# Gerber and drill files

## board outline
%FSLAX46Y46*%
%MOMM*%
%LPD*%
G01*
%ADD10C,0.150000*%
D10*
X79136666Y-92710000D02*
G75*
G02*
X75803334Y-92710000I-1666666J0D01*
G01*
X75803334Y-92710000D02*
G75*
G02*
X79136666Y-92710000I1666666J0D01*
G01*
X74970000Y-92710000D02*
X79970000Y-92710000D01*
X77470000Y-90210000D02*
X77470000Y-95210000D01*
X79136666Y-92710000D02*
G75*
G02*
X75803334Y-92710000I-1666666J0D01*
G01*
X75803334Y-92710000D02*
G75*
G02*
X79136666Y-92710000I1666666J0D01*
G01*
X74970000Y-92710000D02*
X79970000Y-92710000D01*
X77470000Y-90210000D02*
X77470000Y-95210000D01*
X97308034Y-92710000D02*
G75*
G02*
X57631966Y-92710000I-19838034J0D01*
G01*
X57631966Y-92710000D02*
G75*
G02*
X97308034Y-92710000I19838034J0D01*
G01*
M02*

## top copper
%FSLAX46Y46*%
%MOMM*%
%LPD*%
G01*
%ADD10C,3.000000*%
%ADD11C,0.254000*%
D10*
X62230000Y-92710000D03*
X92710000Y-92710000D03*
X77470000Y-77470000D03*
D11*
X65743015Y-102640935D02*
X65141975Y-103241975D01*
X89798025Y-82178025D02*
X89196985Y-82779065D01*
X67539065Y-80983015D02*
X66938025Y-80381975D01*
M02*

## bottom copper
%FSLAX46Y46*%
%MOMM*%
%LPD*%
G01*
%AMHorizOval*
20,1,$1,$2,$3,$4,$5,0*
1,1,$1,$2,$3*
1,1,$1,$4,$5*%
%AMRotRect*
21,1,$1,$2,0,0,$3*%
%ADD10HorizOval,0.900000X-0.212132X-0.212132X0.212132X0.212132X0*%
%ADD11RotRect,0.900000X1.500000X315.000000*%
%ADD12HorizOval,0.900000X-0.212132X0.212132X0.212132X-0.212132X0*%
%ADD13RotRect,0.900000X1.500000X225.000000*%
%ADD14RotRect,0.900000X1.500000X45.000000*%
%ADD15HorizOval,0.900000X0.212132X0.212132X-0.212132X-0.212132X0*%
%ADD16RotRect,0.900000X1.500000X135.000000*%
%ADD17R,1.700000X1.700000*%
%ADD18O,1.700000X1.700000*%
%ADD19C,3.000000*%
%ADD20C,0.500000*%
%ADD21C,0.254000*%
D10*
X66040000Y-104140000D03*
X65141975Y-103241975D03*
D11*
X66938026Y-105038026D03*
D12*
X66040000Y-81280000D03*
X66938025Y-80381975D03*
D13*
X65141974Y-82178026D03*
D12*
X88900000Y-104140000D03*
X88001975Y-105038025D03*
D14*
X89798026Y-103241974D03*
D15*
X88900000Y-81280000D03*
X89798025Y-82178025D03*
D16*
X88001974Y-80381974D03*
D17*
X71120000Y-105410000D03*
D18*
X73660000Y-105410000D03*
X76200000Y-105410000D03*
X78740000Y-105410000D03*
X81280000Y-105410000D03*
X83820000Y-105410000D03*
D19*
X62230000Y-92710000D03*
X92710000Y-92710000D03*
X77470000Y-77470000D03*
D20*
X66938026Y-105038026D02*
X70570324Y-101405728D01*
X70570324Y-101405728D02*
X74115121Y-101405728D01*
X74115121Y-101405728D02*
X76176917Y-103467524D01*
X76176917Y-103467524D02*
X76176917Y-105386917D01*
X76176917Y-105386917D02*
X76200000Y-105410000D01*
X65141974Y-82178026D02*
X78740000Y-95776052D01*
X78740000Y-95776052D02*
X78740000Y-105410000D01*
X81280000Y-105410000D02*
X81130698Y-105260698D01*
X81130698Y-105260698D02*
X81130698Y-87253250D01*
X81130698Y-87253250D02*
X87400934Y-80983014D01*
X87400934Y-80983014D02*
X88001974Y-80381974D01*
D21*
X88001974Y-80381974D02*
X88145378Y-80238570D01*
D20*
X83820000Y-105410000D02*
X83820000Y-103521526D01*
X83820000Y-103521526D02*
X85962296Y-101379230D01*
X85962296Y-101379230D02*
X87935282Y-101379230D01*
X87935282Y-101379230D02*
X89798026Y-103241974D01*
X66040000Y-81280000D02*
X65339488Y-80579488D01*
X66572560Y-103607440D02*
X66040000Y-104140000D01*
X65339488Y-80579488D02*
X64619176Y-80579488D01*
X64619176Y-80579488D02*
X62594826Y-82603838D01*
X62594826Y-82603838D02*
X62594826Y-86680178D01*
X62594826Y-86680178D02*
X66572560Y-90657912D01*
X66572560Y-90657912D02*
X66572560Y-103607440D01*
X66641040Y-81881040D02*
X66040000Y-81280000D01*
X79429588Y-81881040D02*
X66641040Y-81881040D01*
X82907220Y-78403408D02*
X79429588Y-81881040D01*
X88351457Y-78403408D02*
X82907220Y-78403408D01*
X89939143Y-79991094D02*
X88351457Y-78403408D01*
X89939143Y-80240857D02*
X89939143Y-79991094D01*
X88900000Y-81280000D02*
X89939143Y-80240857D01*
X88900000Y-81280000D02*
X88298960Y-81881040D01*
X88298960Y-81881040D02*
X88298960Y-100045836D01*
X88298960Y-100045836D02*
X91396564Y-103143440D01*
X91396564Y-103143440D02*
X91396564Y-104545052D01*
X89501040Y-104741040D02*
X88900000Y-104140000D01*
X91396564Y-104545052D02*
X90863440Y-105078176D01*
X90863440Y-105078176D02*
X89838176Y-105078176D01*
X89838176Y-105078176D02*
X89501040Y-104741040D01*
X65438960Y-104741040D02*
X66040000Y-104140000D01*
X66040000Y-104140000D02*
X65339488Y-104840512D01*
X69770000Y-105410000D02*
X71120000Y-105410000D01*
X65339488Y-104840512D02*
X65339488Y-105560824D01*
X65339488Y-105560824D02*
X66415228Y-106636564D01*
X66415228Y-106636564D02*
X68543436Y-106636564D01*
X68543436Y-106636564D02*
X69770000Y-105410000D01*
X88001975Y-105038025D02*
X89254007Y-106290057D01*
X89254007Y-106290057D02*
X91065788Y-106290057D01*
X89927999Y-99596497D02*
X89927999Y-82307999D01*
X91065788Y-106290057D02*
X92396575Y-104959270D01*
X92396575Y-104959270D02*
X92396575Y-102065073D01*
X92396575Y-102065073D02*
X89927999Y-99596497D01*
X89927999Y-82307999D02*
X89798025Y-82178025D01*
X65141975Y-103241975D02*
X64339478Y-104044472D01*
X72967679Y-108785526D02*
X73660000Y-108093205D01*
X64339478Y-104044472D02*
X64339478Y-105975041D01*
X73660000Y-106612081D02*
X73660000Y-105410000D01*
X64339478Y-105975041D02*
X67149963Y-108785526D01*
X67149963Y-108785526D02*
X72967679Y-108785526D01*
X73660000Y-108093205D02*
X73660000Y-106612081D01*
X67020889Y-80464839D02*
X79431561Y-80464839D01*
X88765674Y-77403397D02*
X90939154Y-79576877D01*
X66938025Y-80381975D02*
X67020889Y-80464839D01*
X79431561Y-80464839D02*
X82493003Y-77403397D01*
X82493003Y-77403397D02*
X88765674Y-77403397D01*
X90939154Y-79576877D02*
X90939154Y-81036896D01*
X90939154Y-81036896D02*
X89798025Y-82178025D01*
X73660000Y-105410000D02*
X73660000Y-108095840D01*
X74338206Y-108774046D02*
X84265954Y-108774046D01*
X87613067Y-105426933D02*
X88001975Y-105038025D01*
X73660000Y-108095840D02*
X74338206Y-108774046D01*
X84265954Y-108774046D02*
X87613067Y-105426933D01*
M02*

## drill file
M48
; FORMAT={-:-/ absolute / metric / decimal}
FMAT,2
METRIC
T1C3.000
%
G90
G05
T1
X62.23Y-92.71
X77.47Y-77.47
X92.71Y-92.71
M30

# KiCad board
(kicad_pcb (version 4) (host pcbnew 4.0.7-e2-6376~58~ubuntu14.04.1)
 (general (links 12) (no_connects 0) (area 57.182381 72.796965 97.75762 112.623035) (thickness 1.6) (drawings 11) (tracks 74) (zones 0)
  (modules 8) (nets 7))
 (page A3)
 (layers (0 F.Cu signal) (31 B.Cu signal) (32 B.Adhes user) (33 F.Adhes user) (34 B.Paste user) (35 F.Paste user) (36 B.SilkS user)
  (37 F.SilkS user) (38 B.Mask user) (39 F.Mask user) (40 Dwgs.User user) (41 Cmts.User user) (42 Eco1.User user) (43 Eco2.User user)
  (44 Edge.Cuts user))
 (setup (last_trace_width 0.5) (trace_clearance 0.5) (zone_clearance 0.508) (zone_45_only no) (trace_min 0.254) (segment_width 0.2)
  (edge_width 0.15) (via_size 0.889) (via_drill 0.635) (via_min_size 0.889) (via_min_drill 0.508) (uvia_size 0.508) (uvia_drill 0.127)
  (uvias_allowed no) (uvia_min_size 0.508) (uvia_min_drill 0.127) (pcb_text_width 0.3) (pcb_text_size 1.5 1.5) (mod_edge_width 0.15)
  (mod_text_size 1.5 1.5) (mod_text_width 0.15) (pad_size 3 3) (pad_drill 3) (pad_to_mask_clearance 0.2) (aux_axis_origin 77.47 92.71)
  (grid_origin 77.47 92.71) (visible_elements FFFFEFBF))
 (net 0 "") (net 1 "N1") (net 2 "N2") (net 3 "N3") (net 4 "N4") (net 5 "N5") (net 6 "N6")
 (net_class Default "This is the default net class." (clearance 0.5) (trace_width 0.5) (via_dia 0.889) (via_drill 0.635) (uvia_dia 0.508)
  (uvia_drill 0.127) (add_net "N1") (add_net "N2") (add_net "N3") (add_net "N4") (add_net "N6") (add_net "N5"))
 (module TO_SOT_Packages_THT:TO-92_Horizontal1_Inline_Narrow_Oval (layer F.Cu) (at 66.938026 105.038026 135)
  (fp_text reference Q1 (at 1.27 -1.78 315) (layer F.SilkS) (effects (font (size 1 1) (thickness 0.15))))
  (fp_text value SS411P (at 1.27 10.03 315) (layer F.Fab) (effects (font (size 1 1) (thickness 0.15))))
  (pad 2 smd oval (at 1.270001 0 315) (size 0.9 1.5) (layers B.Cu F.Paste F.Mask) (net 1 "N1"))
  (pad 3 smd oval (at 2.54 0 315) (size 0.9 1.5) (layers B.Cu F.Paste F.Mask) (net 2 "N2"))
  (pad 1 smd rect (at 0 0 315) (size 0.9 1.5) (layers B.Cu F.Paste F.Mask) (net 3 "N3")))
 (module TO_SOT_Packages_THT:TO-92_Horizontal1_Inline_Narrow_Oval (layer F.Cu) (at 65.141974 82.178026 45)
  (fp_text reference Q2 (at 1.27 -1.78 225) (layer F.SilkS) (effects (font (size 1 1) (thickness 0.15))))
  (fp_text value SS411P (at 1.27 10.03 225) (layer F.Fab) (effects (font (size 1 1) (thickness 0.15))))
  (pad 2 smd oval (at 1.270001 0 225) (size 0.9 1.5) (layers B.Cu F.Paste F.Mask) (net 1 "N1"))
  (pad 3 smd oval (at 2.54 0 225) (size 0.9 1.5) (layers B.Cu F.Paste F.Mask) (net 2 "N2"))
  (pad 1 smd rect (at 0 0 225) (size 0.9 1.5) (layers B.Cu F.Paste F.Mask) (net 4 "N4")))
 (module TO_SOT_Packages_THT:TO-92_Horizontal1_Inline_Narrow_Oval (layer F.Cu) (at 89.798026 103.241974 225)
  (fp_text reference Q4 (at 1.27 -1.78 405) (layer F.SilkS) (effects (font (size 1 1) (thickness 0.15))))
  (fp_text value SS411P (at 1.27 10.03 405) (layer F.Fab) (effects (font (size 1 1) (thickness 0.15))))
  (pad 2 smd oval (at 1.270001 0 45) (size 0.9 1.5) (layers B.Cu F.Paste F.Mask) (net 1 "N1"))
  (pad 3 smd oval (at 2.54 0 45) (size 0.9 1.5) (layers B.Cu F.Paste F.Mask) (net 2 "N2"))
  (pad 1 smd rect (at 0 0 45) (size 0.9 1.5) (layers B.Cu F.Paste F.Mask) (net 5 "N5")))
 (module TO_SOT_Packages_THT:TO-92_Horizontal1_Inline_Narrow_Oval (layer F.Cu) (at 88.001974 80.381974 315)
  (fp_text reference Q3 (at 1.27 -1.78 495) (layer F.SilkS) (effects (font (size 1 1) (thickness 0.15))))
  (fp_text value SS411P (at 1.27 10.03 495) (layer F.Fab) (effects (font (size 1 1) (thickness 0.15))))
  (pad 2 smd oval (at 1.270001 0 135) (size 0.9 1.5) (layers B.Cu F.Paste F.Mask) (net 1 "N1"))
  (pad 3 smd oval (at 2.54 0 135) (size 0.9 1.5) (layers B.Cu F.Paste F.Mask) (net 2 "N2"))
  (pad 1 smd rect (at 0 0 135) (size 0.9 1.5) (layers B.Cu F.Paste F.Mask) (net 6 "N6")))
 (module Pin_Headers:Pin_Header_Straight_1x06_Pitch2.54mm (layer B.Cu) (at 71.12 105.41 270)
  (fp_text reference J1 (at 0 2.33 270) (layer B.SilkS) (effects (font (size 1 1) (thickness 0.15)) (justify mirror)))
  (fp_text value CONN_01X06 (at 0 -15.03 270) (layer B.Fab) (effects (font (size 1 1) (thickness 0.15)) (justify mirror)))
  (pad 1 smd rect (at 0 0 270) (size 1.7 1.7) (layers B.Cu B.Paste B.Mask) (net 1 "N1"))
  (pad 2 smd oval (at 0 -2.54 270) (size 1.7 1.7) (layers B.Cu B.Paste B.Mask) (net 2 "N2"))
  (pad 3 smd oval (at 0 -5.08 270) (size 1.7 1.7) (layers B.Cu B.Paste B.Mask) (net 3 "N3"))
  (pad 4 smd oval (at 0 -7.62 270) (size 1.7 1.7) (layers B.Cu B.Paste B.Mask) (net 4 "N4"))
  (pad 5 smd oval (at 0 -10.16 270) (size 1.7 1.7) (layers B.Cu B.Paste B.Mask) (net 6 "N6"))
  (pad 6 smd oval (at 0 -12.7 270) (size 1.7 1.7) (layers B.Cu B.Paste B.Mask) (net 5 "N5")))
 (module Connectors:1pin (layer F.Cu) (at 62.23 92.71)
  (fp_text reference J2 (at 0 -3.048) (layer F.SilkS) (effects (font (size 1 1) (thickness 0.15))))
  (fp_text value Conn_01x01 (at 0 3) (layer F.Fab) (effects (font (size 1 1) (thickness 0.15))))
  (pad 1 thru_hole circle (at 0 0) (size 3 3) (drill 3) (layers *.Cu *.Mask)))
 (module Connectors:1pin (layer F.Cu) (at 92.71 92.71)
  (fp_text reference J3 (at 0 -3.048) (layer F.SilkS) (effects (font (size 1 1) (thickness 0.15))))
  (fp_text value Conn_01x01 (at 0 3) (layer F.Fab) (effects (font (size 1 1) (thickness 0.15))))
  (pad 1 thru_hole circle (at 0 0) (size 3 3) (drill 3) (layers *.Cu *.Mask)))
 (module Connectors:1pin (layer F.Cu) (at 77.47 77.47)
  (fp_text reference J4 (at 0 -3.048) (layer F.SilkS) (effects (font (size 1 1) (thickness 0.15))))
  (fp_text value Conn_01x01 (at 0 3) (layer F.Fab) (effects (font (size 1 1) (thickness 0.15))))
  (pad 1 thru_hole circle (at 0 0) (size 3 3) (drill 3) (layers *.Cu *.Mask)))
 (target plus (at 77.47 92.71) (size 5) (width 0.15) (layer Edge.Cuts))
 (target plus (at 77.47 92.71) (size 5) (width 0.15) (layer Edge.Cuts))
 (gr_circle (center 77.47 92.71) (end 92.71 105.41) (layer Edge.Cuts) (width 0.15))
 (segment (start 65.743015 102.640935) (end 65.141975 103.241975) (width 0.254) (layer F.Cu) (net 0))
 (segment (start 89.798025 82.178025) (end 89.196985 82.779065) (width 0.254) (layer F.Cu) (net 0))
 (segment (start 67.539065 80.983015) (end 66.938025 80.381975) (width 0.254) (layer F.Cu) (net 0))
 (segment (start 66.938026 105.038026) (end 70.570324 101.405728) (width 0.5) (layer B.Cu) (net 3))
 (segment (start 70.570324 101.405728) (end 74.115121 101.405728) (width 0.5) (layer B.Cu) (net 3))
 (segment (start 74.115121 101.405728) (end 76.176917 103.467524) (width 0.5) (layer B.Cu) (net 3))
 (segment (start 76.176917 103.467524) (end 76.176917 105.386917) (width 0.5) (layer B.Cu) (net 3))
 (segment (start 76.176917 105.386917) (end 76.2 105.41) (width 0.5) (layer B.Cu) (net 3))
 (segment (start 65.141974 82.178026) (end 78.74 95.776052) (width 0.5) (layer B.Cu) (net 4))
 (segment (start 78.74 95.776052) (end 78.74 105.41) (width 0.5) (layer B.Cu) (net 4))
 (segment (start 81.28 105.41) (end 81.130698 105.260698) (width 0.5) (layer B.Cu) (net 6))
 (segment (start 81.130698 105.260698) (end 81.130698 87.25325) (width 0.5) (layer B.Cu) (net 6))
 (segment (start 81.130698 87.25325) (end 87.400934 80.983014) (width 0.5) (layer B.Cu) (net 6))
 (segment (start 87.400934 80.983014) (end 88.001974 80.381974) (width 0.5) (layer B.Cu) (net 6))
 (segment (start 88.001974 80.381974) (end 88.145378 80.23857) (width 0.254) (layer B.Cu) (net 6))
 (segment (start 83.82 105.41) (end 83.82 103.521526) (width 0.5) (layer B.Cu) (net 5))
 (segment (start 83.82 103.521526) (end 85.962296 101.37923) (width 0.5) (layer B.Cu) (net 5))
 (segment (start 85.962296 101.37923) (end 87.935282 101.37923) (width 0.5) (layer B.Cu) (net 5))
 (segment (start 87.935282 101.37923) (end 89.798026 103.241974) (width 0.5) (layer B.Cu) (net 5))
 (segment (start 66.04 81.28) (end 65.339488 80.579488) (width 0.5) (layer B.Cu) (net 1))
 (segment (start 66.57256 103.60744) (end 66.04 104.14) (width 0.5) (layer B.Cu) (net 1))
 (segment (start 65.339488 80.579488) (end 64.619176 80.579488) (width 0.5) (layer B.Cu) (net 1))
 (segment (start 64.619176 80.579488) (end 62.594826 82.603838) (width 0.5) (layer B.Cu) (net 1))
 (segment (start 62.594826 82.603838) (end 62.594826 86.680178) (width 0.5) (layer B.Cu) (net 1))
 (segment (start 62.594826 86.680178) (end 66.57256 90.657912) (width 0.5) (layer B.Cu) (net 1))
 (segment (start 66.57256 90.657912) (end 66.57256 103.60744) (width 0.5) (layer B.Cu) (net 1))
 (segment (start 66.64104 81.88104) (end 66.04 81.28) (width 0.5) (layer B.Cu) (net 1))
 (segment (start 79.429588 81.88104) (end 66.64104 81.88104) (width 0.5) (layer B.Cu) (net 1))
 (segment (start 82.90722 78.403408) (end 79.429588 81.88104) (width 0.5) (layer B.Cu) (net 1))
 (segment (start 88.351457 78.403408) (end 82.90722 78.403408) (width 0.5) (layer B.Cu) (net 1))
 (segment (start 89.939143 79.991094) (end 88.351457 78.403408) (width 0.5) (layer B.Cu) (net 1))
 (segment (start 89.939143 80.240857) (end 89.939143 79.991094) (width 0.5) (layer B.Cu) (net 1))
 (segment (start 88.9 81.28) (end 89.939143 80.240857) (width 0.5) (layer B.Cu) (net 1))
 (segment (start 88.9 81.28) (end 88.29896 81.88104) (width 0.5) (layer B.Cu) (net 1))
 (segment (start 88.29896 81.88104) (end 88.29896 100.045836) (width 0.5) (layer B.Cu) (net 1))
 (segment (start 88.29896 100.045836) (end 91.396564 103.14344) (width 0.5) (layer B.Cu) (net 1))
 (segment (start 91.396564 103.14344) (end 91.396564 104.545052) (width 0.5) (layer B.Cu) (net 1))
 (segment (start 89.50104 104.74104) (end 88.9 104.14) (width 0.5) (layer B.Cu) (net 1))
 (segment (start 91.396564 104.545052) (end 90.86344 105.078176) (width 0.5) (layer B.Cu) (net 1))
 (segment (start 90.86344 105.078176) (end 89.838176 105.078176) (width 0.5) (layer B.Cu) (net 1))
 (segment (start 89.838176 105.078176) (end 89.50104 104.74104) (width 0.5) (layer B.Cu) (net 1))
 (segment (start 65.43896 104.74104) (end 66.04 104.14) (width 0.5) (layer B.Cu) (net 1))
 (segment (start 66.04 104.14) (end 65.339488 104.840512) (width 0.5) (layer B.Cu) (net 1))
 (segment (start 69.77 105.41) (end 71.12 105.41) (width 0.5) (layer B.Cu) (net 1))
 (segment (start 65.339488 104.840512) (end 65.339488 105.560824) (width 0.5) (layer B.Cu) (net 1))
 (segment (start 65.339488 105.560824) (end 66.415228 106.636564) (width 0.5) (layer B.Cu) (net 1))
 (segment (start 66.415228 106.636564) (end 68.543436 106.636564) (width 0.5) (layer B.Cu) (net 1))
 (segment (start 68.543436 106.636564) (end 69.77 105.41) (width 0.5) (layer B.Cu) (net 1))
 (segment (start 88.001975 105.038025) (end 89.254007 106.290057) (width 0.5) (layer B.Cu) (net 2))
 (segment (start 89.254007 106.290057) (end 91.065788 106.290057) (width 0.5) (layer B.Cu) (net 2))
 (segment (start 89.927999 99.596497) (end 89.927999 82.307999) (width 0.5) (layer B.Cu) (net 2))
 (segment (start 91.065788 106.290057) (end 92.396575 104.95927) (width 0.5) (layer B.Cu) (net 2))
 (segment (start 92.396575 104.95927) (end 92.396575 102.065073) (width 0.5) (layer B.Cu) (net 2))
 (segment (start 92.396575 102.065073) (end 89.927999 99.596497) (width 0.5) (layer B.Cu) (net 2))
 (segment (start 89.927999 82.307999) (end 89.798025 82.178025) (width 0.5) (layer B.Cu) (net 2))
 (segment (start 65.141975 103.241975) (end 64.339478 104.044472) (width 0.5) (layer B.Cu) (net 2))
 (segment (start 72.967679 108.785526) (end 73.66 108.093205) (width 0.5) (layer B.Cu) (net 2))
 (segment (start 64.339478 104.044472) (end 64.339478 105.975041) (width 0.5) (layer B.Cu) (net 2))
 (segment (start 73.66 106.612081) (end 73.66 105.41) (width 0.5) (layer B.Cu) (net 2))
 (segment (start 64.339478 105.975041) (end 67.149963 108.785526) (width 0.5) (layer B.Cu) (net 2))
 (segment (start 67.149963 108.785526) (end 72.967679 108.785526) (width 0.5) (layer B.Cu) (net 2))
 (segment (start 73.66 108.093205) (end 73.66 106.612081) (width 0.5) (layer B.Cu) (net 2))
 (segment (start 67.020889 80.464839) (end 79.431561 80.464839) (width 0.5) (layer B.Cu) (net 2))
 (segment (start 88.765674 77.403397) (end 90.939154 79.576877) (width 0.5) (layer B.Cu) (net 2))
 (segment (start 66.938025 80.381975) (end 67.020889 80.464839) (width 0.5) (layer B.Cu) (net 2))
 (segment (start 79.431561 80.464839) (end 82.493003 77.403397) (width 0.5) (layer B.Cu) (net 2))
 (segment (start 82.493003 77.403397) (end 88.765674 77.403397) (width 0.5) (layer B.Cu) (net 2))
 (segment (start 90.939154 79.576877) (end 90.939154 81.036896) (width 0.5) (layer B.Cu) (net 2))
 (segment (start 90.939154 81.036896) (end 89.798025 82.178025) (width 0.5) (layer B.Cu) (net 2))
 (segment (start 73.66 105.41) (end 73.66 108.09584) (width 0.5) (layer B.Cu) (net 2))
 (segment (start 74.338206 108.774046) (end 84.265954 108.774046) (width 0.5) (layer B.Cu) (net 2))
 (segment (start 87.613067 105.426933) (end 88.001975 105.038025) (width 0.5) (layer B.Cu) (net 2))
 (segment (start 73.66 108.09584) (end 74.338206 108.774046) (width 0.5) (layer B.Cu) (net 2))
 (segment (start 84.265954 108.774046) (end 87.613067 105.426933) (width 0.5) (layer B.Cu) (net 2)))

